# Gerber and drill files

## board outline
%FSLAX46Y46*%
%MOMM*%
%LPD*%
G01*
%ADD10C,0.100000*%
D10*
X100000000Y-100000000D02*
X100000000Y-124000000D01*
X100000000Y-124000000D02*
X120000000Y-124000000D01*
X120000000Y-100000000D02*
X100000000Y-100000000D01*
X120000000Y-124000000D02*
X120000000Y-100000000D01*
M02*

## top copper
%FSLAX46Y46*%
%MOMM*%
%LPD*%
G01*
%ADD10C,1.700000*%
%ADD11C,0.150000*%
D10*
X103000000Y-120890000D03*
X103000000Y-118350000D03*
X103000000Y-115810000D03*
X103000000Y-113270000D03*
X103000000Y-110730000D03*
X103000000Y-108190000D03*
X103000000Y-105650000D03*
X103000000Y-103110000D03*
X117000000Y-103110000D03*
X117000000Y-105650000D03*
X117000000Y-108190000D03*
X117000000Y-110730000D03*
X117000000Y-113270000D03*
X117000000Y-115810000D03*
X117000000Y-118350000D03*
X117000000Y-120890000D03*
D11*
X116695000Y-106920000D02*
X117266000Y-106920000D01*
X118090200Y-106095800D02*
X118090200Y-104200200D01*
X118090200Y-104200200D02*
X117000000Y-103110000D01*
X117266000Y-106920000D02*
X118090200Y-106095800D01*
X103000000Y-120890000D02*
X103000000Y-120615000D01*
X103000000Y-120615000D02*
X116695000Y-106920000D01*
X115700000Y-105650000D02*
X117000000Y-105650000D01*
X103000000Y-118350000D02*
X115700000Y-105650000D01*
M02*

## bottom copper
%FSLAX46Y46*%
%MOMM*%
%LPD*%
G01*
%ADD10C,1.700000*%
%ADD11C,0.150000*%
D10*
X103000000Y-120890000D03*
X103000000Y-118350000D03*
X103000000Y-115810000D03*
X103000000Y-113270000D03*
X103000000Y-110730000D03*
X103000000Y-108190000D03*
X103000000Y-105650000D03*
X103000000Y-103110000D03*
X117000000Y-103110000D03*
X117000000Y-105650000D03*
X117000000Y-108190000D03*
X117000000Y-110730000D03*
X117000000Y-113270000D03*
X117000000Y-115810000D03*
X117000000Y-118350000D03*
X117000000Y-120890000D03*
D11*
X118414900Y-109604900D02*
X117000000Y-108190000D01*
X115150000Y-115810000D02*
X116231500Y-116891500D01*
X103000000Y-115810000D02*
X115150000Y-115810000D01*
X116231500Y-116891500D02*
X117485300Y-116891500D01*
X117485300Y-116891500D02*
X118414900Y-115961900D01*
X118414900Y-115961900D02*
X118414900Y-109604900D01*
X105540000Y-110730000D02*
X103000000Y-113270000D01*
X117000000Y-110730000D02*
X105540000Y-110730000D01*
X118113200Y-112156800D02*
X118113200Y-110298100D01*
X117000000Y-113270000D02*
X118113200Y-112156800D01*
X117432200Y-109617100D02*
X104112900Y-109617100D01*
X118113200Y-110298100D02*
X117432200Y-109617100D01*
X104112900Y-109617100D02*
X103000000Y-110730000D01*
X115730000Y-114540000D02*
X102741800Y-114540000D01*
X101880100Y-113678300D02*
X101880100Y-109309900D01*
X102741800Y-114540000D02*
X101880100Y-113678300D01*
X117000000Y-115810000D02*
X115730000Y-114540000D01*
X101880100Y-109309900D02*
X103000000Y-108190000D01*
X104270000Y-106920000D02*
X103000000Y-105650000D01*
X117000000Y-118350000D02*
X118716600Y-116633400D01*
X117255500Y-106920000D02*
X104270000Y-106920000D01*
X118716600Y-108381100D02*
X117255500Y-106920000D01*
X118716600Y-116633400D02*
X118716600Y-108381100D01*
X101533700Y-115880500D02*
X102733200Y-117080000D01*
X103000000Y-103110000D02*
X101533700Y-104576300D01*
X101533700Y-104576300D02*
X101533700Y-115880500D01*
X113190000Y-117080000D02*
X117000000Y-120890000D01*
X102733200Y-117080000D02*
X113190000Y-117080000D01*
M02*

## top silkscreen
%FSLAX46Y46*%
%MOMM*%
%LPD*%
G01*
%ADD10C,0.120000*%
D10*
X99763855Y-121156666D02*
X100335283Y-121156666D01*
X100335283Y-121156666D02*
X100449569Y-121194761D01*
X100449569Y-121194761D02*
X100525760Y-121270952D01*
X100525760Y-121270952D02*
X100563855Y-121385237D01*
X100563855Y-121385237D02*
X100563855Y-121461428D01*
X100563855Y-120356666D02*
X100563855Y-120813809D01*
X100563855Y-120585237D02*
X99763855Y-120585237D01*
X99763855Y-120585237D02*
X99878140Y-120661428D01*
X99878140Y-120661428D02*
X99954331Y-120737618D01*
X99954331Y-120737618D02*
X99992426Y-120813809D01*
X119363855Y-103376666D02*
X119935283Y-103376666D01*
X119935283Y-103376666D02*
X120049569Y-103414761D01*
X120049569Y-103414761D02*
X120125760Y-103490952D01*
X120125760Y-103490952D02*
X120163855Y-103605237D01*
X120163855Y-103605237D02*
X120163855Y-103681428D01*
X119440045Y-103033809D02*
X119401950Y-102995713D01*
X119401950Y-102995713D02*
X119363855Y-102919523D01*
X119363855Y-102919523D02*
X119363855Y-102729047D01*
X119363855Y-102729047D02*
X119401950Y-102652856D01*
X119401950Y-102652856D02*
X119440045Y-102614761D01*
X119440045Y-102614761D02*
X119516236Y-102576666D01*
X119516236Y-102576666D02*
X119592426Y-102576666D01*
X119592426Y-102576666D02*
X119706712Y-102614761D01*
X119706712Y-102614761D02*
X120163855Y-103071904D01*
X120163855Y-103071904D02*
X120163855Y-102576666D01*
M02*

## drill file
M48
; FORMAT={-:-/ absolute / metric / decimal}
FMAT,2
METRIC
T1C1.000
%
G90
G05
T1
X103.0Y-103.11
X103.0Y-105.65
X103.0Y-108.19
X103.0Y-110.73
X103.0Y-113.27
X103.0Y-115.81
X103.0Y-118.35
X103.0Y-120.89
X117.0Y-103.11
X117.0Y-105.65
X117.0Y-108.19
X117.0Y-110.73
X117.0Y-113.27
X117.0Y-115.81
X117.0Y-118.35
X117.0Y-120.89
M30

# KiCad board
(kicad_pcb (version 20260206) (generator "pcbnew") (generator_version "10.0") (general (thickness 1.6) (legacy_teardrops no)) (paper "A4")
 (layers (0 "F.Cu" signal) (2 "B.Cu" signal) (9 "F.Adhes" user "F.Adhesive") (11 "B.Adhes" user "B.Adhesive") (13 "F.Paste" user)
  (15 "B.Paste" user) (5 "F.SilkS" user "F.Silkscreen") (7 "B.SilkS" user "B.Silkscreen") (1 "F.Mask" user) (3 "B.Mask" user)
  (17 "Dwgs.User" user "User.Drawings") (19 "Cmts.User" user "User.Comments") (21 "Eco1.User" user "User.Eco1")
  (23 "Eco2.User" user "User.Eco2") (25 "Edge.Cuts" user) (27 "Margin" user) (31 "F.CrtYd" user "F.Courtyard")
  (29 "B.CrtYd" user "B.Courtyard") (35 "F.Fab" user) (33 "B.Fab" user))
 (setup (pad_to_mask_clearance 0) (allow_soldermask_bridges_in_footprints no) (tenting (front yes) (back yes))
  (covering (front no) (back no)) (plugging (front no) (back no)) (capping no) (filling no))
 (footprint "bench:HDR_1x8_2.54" (layer "F.Cu") (at 103 120.89 90)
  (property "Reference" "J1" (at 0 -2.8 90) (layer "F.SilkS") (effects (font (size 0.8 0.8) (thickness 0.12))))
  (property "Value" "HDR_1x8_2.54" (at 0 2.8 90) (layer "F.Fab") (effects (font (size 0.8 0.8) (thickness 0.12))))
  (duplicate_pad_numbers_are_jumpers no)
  (pad "1" thru_hole circle (at 0 0 90) (size 1.7 1.7) (drill 1) (layers "*.Cu" "*.Mask") (remove_unused_layers no) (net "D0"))
  (pad "2" thru_hole circle (at 2.54 0 90) (size 1.7 1.7) (drill 1) (layers "*.Cu" "*.Mask") (remove_unused_layers no) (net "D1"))
  (pad "3" thru_hole circle (at 5.08 0 90) (size 1.7 1.7) (drill 1) (layers "*.Cu" "*.Mask") (remove_unused_layers no) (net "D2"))
  (pad "4" thru_hole circle (at 7.62 0 90) (size 1.7 1.7) (drill 1) (layers "*.Cu" "*.Mask") (remove_unused_layers no) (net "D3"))
  (pad "5" thru_hole circle (at 10.16 0 90) (size 1.7 1.7) (drill 1) (layers "*.Cu" "*.Mask") (remove_unused_layers no) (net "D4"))
  (pad "6" thru_hole circle (at 12.7 0 90) (size 1.7 1.7) (drill 1) (layers "*.Cu" "*.Mask") (remove_unused_layers no) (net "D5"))
  (pad "7" thru_hole circle (at 15.24 0 90) (size 1.7 1.7) (drill 1) (layers "*.Cu" "*.Mask") (remove_unused_layers no) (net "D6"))
  (pad "8" thru_hole circle (at 17.78 0 90) (size 1.7 1.7) (drill 1) (layers "*.Cu" "*.Mask") (remove_unused_layers no) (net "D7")))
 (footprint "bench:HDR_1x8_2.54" (layer "F.Cu") (at 117 103.11 -90)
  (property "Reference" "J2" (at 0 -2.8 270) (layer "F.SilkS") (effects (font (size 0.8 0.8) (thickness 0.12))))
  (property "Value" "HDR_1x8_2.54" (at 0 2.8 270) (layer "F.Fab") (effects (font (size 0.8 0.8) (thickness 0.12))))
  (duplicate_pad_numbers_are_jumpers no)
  (pad "1" thru_hole circle (at 0 0 270) (size 1.7 1.7) (drill 1) (layers "*.Cu" "*.Mask") (remove_unused_layers no) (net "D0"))
  (pad "2" thru_hole circle (at 2.54 0 270) (size 1.7 1.7) (drill 1) (layers "*.Cu" "*.Mask") (remove_unused_layers no) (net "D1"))
  (pad "3" thru_hole circle (at 5.08 0 270) (size 1.7 1.7) (drill 1) (layers "*.Cu" "*.Mask") (remove_unused_layers no) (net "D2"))
  (pad "4" thru_hole circle (at 7.62 0 270) (size 1.7 1.7) (drill 1) (layers "*.Cu" "*.Mask") (remove_unused_layers no) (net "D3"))
  (pad "5" thru_hole circle (at 10.16 0 270) (size 1.7 1.7) (drill 1) (layers "*.Cu" "*.Mask") (remove_unused_layers no) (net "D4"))
  (pad "6" thru_hole circle (at 12.7 0 270) (size 1.7 1.7) (drill 1) (layers "*.Cu" "*.Mask") (remove_unused_layers no) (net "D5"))
  (pad "7" thru_hole circle (at 15.24 0 270) (size 1.7 1.7) (drill 1) (layers "*.Cu" "*.Mask") (remove_unused_layers no) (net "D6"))
  (pad "8" thru_hole circle (at 17.78 0 270) (size 1.7 1.7) (drill 1) (layers "*.Cu" "*.Mask") (remove_unused_layers no) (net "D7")))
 (gr_line (start 100 100) (end 100 124) (stroke (width 0.1) (type solid)) (layer "Edge.Cuts"))
 (gr_line (start 100 124) (end 120 124) (stroke (width 0.1) (type solid)) (layer "Edge.Cuts"))
 (gr_line (start 120 100) (end 100 100) (stroke (width 0.1) (type solid)) (layer "Edge.Cuts"))
 (gr_line (start 120 124) (end 120 100) (stroke (width 0.1) (type solid)) (layer "Edge.Cuts"))
 (segment (start 116.695 106.92) (end 117.266 106.92) (width 0.15) (layer "F.Cu") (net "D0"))
 (segment (start 118.0902 106.0958) (end 118.0902 104.2002) (width 0.15) (layer "F.Cu") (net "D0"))
 (segment (start 118.0902 104.2002) (end 117 103.11) (width 0.15) (layer "F.Cu") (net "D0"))
 (segment (start 117.266 106.92) (end 118.0902 106.0958) (width 0.15) (layer "F.Cu") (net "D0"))
 (segment (start 103 120.89) (end 103 120.615) (width 0.15) (layer "F.Cu") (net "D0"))
 (segment (start 103 120.615) (end 116.695 106.92) (width 0.15) (layer "F.Cu") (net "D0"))
 (segment (start 115.7 105.65) (end 117 105.65) (width 0.15) (layer "F.Cu") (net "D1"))
 (segment (start 103 118.35) (end 115.7 105.65) (width 0.15) (layer "F.Cu") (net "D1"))
 (segment (start 118.4149 109.6049) (end 117 108.19) (width 0.15) (layer "B.Cu") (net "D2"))
 (segment (start 115.15 115.81) (end 116.2315 116.8915) (width 0.15) (layer "B.Cu") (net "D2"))
 (segment (start 103 115.81) (end 115.15 115.81) (width 0.15) (layer "B.Cu") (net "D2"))
 (segment (start 116.2315 116.8915) (end 117.4853 116.8915) (width 0.15) (layer "B.Cu") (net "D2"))
 (segment (start 117.4853 116.8915) (end 118.4149 115.9619) (width 0.15) (layer "B.Cu") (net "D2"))
 (segment (start 118.4149 115.9619) (end 118.4149 109.6049) (width 0.15) (layer "B.Cu") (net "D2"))
 (segment (start 105.54 110.73) (end 103 113.27) (width 0.15) (layer "B.Cu") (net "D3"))
 (segment (start 117 110.73) (end 105.54 110.73) (width 0.15) (layer "B.Cu") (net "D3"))
 (segment (start 118.1132 112.1568) (end 118.1132 110.2981) (width 0.15) (layer "B.Cu") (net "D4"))
 (segment (start 117 113.27) (end 118.1132 112.1568) (width 0.15) (layer "B.Cu") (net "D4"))
 (segment (start 117.4322 109.6171) (end 104.1129 109.6171) (width 0.15) (layer "B.Cu") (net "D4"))
 (segment (start 118.1132 110.2981) (end 117.4322 109.6171) (width 0.15) (layer "B.Cu") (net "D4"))
 (segment (start 104.1129 109.6171) (end 103 110.73) (width 0.15) (layer "B.Cu") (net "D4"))
 (segment (start 115.73 114.54) (end 102.7418 114.54) (width 0.15) (layer "B.Cu") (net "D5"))
 (segment (start 101.8801 113.6783) (end 101.8801 109.3099) (width 0.15) (layer "B.Cu") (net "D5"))
 (segment (start 102.7418 114.54) (end 101.8801 113.6783) (width 0.15) (layer "B.Cu") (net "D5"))
 (segment (start 117 115.81) (end 115.73 114.54) (width 0.15) (layer "B.Cu") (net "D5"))
 (segment (start 101.8801 109.3099) (end 103 108.19) (width 0.15) (layer "B.Cu") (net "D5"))
 (segment (start 104.27 106.92) (end 103 105.65) (width 0.15) (layer "B.Cu") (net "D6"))
 (segment (start 117 118.35) (end 118.7166 116.6334) (width 0.15) (layer "B.Cu") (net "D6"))
 (segment (start 117.2555 106.92) (end 104.27 106.92) (width 0.15) (layer "B.Cu") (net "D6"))
 (segment (start 118.7166 108.3811) (end 117.2555 106.92) (width 0.15) (layer "B.Cu") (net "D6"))
 (segment (start 118.7166 116.6334) (end 118.7166 108.3811) (width 0.15) (layer "B.Cu") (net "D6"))
 (segment (start 101.5337 115.8805) (end 102.7332 117.08) (width 0.15) (layer "B.Cu") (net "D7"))
 (segment (start 103 103.11) (end 101.5337 104.5763) (width 0.15) (layer "B.Cu") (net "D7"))
 (segment (start 101.5337 104.5763) (end 101.5337 115.8805) (width 0.15) (layer "B.Cu") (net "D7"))
 (segment (start 113.19 117.08) (end 117 120.89) (width 0.15) (layer "B.Cu") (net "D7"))
 (segment (start 102.7332 117.08) (end 113.19 117.08) (width 0.15) (layer "B.Cu") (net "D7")))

